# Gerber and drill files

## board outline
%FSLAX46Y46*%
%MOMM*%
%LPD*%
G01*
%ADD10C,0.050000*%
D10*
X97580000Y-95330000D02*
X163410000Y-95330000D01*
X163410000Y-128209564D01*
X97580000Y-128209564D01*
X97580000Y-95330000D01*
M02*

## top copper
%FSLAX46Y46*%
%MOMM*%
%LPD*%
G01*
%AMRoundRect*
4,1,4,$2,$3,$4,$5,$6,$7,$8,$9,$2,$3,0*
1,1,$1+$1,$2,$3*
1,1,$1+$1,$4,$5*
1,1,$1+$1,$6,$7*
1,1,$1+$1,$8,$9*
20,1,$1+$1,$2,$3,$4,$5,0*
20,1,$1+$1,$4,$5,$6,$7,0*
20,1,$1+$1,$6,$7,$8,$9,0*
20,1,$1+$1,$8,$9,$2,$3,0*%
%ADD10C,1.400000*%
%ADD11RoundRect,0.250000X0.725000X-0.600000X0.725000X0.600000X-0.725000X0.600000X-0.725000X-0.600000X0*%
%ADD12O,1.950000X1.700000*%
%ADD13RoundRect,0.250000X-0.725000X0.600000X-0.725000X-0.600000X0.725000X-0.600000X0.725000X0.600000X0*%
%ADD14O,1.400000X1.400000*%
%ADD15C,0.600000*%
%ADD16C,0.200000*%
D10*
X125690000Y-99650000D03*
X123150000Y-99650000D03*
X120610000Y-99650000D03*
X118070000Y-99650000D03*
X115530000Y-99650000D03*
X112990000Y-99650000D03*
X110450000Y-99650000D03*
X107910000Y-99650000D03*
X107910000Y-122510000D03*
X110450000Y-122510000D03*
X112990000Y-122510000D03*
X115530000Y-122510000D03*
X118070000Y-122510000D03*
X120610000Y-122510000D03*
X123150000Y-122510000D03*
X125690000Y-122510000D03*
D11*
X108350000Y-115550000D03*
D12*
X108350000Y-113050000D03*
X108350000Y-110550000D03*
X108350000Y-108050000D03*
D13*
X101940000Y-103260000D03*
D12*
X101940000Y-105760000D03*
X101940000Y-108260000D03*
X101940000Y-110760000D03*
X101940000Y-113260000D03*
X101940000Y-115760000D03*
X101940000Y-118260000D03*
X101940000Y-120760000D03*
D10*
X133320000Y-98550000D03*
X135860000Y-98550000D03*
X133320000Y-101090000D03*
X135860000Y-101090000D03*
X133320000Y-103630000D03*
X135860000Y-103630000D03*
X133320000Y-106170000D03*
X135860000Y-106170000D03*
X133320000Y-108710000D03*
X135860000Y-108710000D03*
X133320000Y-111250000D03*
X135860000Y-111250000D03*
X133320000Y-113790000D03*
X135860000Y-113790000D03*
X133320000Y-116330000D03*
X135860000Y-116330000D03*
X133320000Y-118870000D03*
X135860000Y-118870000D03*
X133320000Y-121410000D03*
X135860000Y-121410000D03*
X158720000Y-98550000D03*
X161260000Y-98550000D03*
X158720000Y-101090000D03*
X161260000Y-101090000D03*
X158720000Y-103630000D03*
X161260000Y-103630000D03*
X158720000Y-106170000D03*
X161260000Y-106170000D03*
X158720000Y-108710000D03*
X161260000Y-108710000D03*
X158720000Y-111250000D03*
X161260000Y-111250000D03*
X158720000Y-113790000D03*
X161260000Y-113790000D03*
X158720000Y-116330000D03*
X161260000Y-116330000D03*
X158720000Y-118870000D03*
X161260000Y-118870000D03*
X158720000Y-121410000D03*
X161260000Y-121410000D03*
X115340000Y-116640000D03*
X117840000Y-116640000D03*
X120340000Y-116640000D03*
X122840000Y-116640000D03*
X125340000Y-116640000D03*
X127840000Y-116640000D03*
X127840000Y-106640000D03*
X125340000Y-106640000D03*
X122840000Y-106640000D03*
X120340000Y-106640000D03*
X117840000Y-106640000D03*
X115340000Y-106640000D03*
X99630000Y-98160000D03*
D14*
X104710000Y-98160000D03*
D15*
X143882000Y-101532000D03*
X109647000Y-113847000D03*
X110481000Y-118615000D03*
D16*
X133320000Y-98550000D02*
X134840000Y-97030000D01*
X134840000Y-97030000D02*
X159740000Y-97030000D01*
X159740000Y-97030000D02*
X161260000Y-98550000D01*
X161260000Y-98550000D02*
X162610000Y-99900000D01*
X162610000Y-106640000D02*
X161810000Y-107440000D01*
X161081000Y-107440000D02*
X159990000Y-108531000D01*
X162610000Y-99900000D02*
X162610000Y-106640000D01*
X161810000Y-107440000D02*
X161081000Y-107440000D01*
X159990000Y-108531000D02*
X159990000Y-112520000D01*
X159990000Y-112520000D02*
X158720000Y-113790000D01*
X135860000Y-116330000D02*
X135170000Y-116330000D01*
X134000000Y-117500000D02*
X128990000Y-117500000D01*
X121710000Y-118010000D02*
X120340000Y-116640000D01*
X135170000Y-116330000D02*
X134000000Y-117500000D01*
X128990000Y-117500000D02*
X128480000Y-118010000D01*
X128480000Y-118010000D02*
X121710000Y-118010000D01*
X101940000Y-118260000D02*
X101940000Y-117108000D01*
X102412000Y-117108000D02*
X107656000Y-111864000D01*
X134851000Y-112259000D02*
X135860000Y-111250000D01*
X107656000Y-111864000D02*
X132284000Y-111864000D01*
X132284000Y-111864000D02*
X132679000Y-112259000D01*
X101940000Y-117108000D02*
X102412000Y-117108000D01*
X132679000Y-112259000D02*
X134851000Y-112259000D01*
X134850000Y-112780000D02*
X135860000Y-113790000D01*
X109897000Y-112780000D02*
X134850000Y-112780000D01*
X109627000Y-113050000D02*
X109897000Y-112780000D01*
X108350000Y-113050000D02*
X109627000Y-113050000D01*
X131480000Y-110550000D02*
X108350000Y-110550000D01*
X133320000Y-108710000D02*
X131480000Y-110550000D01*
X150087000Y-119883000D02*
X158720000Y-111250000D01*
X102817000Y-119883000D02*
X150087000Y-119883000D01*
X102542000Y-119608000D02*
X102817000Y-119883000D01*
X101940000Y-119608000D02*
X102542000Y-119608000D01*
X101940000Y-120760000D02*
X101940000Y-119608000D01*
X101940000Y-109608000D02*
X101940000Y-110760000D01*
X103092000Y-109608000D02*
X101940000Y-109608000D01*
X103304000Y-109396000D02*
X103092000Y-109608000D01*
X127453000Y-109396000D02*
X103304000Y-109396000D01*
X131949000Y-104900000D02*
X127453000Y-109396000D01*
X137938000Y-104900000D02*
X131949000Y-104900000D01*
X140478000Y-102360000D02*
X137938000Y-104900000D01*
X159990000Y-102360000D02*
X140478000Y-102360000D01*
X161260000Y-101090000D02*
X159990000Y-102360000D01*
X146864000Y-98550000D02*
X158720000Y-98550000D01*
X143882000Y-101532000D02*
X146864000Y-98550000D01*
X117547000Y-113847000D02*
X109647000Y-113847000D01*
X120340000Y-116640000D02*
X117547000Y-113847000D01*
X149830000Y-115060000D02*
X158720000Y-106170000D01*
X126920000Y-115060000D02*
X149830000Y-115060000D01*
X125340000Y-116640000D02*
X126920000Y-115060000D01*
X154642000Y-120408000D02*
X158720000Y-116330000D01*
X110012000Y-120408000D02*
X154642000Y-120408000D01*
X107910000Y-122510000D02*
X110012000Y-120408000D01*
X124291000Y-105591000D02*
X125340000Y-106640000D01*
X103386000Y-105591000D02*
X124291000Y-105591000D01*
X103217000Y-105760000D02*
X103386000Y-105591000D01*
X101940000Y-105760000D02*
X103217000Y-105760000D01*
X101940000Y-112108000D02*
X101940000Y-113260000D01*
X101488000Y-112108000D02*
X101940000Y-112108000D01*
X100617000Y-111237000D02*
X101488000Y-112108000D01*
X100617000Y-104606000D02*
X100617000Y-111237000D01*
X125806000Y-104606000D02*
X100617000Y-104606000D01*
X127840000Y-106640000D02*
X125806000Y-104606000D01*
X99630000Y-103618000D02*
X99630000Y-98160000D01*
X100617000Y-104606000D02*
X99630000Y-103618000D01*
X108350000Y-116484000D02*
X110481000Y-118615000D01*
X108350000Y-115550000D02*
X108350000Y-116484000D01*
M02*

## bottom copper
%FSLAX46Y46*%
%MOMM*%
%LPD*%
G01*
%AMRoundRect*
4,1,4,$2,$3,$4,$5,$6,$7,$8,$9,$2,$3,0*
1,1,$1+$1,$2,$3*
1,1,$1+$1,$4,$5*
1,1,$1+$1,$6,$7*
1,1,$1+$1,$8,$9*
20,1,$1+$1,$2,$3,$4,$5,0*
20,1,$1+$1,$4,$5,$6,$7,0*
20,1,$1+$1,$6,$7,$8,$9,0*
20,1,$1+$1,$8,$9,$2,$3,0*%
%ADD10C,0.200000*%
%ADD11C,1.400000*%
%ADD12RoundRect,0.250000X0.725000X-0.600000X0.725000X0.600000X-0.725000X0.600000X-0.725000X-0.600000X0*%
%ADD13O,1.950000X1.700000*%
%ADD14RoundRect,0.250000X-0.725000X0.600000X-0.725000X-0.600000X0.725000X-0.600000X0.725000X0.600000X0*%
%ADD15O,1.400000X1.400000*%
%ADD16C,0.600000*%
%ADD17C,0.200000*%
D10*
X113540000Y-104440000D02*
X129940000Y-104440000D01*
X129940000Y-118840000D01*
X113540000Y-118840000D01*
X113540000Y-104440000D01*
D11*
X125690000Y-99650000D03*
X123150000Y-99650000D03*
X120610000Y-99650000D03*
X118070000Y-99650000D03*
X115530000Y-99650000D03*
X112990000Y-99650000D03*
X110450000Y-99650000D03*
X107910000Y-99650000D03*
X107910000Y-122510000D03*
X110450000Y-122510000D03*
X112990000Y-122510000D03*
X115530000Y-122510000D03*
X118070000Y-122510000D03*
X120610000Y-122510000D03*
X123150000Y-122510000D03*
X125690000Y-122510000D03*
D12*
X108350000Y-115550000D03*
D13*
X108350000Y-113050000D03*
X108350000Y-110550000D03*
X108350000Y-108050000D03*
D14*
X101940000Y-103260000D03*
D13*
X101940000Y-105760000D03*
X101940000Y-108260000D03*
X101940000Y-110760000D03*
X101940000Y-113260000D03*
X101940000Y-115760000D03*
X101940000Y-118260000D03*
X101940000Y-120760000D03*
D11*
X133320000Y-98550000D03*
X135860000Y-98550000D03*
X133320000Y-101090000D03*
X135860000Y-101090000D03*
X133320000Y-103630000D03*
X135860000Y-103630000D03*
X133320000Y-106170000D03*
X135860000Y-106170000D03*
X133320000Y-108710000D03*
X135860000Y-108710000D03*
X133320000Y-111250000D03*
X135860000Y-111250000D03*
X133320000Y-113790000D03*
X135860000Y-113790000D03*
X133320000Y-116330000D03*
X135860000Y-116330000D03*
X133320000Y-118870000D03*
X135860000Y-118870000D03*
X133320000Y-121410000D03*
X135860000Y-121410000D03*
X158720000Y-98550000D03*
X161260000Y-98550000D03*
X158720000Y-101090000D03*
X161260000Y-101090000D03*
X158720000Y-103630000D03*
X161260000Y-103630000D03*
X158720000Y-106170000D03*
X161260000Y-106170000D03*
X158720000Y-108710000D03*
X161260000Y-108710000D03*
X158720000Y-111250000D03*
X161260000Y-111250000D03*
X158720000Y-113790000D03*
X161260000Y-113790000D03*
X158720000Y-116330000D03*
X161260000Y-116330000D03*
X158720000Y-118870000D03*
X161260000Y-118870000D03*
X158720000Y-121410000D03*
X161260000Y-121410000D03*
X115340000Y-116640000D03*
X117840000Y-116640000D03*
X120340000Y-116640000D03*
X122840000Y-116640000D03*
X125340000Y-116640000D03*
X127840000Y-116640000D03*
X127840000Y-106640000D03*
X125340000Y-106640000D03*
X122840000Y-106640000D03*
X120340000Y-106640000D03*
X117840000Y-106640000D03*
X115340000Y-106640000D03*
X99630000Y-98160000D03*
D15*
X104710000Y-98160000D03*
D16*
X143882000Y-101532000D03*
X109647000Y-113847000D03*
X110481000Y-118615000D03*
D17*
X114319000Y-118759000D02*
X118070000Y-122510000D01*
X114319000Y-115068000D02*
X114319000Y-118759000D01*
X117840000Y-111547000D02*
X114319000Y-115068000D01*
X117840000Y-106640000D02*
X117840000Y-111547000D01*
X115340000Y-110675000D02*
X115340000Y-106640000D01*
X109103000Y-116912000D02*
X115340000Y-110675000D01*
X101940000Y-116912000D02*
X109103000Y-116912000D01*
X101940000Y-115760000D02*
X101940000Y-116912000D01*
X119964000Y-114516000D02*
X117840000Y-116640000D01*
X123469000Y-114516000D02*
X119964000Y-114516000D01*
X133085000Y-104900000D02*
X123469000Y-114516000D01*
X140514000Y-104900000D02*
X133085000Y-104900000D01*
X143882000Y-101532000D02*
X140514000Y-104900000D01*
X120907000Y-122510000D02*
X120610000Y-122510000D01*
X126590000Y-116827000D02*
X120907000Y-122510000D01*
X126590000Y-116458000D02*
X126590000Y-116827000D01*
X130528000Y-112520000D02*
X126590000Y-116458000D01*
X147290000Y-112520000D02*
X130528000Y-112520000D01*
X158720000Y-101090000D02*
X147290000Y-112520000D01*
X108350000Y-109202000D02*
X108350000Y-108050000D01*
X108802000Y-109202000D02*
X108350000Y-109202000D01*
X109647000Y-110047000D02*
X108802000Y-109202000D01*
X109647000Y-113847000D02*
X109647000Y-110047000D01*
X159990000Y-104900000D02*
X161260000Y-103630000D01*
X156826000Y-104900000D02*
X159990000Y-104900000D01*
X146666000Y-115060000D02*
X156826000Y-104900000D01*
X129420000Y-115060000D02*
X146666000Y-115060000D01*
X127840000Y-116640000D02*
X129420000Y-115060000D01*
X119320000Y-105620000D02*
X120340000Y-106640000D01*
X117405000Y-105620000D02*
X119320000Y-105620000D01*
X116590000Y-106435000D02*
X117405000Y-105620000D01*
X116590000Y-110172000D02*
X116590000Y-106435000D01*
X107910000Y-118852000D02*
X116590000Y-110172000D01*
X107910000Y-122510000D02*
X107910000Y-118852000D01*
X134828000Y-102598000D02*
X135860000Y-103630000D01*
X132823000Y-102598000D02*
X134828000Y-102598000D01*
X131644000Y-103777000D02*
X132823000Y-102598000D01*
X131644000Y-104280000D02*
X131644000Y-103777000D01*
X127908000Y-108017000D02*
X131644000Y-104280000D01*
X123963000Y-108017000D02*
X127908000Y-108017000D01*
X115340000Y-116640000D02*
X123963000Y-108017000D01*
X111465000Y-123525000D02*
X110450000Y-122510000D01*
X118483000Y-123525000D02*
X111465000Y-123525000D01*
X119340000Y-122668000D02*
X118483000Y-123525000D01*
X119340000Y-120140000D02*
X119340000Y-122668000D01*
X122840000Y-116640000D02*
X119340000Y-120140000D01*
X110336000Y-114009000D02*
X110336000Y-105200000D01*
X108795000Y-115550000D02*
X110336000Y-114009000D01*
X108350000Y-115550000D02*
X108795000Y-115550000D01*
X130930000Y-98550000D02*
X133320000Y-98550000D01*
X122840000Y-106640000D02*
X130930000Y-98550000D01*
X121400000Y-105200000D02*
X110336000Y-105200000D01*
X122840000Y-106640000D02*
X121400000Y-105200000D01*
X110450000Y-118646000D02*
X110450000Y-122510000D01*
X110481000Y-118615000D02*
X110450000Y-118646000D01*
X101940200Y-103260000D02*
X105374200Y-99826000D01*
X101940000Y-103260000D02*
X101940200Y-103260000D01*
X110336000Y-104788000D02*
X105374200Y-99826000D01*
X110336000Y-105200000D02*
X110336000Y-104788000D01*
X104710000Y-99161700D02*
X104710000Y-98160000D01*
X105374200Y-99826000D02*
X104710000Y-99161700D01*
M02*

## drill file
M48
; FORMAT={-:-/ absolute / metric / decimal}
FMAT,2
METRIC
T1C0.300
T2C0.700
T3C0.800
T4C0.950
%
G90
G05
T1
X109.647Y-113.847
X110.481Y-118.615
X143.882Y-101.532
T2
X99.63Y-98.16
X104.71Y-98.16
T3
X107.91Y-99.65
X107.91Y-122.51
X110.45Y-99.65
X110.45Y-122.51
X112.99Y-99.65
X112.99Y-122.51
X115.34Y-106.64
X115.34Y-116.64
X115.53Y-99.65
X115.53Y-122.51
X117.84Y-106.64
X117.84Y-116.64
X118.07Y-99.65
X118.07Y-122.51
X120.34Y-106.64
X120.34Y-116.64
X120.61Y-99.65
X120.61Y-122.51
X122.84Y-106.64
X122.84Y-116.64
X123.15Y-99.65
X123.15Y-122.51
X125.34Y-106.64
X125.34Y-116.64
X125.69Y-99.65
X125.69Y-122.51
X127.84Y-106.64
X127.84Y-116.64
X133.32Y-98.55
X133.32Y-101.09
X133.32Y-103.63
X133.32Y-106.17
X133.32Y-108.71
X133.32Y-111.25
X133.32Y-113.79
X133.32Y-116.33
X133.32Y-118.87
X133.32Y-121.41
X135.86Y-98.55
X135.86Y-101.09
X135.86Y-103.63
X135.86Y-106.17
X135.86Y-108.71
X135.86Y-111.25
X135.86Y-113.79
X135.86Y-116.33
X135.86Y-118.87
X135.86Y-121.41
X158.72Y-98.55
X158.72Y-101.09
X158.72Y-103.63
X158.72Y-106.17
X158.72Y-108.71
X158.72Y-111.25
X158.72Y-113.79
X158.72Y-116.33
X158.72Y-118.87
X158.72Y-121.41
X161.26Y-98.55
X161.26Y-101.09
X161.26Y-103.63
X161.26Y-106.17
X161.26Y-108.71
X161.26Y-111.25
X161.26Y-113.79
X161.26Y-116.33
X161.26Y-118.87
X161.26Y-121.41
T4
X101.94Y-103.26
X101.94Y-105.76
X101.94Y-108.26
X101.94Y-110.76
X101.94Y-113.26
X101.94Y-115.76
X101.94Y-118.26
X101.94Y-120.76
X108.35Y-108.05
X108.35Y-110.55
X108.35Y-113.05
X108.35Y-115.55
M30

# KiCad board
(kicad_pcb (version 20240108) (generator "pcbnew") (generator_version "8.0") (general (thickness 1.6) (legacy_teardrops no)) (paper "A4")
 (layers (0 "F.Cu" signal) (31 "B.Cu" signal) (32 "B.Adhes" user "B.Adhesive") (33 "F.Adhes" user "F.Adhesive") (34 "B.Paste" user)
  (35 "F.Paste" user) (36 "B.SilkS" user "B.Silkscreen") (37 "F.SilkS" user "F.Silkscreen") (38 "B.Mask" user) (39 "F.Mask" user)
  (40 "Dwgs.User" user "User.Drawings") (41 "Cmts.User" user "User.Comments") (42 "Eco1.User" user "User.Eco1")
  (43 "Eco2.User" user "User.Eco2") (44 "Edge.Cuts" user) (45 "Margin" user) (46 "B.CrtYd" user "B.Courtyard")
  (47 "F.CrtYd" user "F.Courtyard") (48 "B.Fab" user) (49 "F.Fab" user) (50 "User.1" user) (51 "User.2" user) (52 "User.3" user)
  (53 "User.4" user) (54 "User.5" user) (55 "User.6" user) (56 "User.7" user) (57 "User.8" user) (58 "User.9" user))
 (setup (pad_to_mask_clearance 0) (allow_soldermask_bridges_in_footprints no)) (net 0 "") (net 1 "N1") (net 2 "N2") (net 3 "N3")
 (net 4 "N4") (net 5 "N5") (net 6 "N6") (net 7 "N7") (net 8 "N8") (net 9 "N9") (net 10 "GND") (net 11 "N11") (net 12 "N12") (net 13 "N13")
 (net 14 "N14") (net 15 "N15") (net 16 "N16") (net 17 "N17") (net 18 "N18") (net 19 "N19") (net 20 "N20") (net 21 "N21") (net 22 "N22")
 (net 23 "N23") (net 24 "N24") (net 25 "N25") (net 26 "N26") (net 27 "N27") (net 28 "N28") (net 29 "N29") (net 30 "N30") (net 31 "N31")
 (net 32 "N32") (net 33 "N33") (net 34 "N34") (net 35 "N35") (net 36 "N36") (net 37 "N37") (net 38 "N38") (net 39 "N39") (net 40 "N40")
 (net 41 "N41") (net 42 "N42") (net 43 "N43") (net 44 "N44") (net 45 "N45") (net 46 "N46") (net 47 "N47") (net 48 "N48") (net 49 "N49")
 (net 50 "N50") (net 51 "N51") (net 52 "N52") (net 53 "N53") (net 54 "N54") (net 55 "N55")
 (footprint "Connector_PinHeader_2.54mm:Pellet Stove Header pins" (layer "F.Cu") (at 114.26 111.08 -90)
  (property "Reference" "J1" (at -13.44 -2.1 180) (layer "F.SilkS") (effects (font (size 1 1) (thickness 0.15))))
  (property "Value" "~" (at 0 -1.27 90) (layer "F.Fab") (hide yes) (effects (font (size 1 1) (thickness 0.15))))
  (pad "1" thru_hole circle (at -11.43 -11.43 180) (size 1.4 1.4) (drill 0.8) (layers "*.Cu" "*.Mask") (remove_unused_layers no)
   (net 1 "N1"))
  (pad "2" thru_hole circle (at -11.43 -8.89 180) (size 1.4 1.4) (drill 0.8) (layers "*.Cu" "*.Mask") (remove_unused_layers no) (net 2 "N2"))
  (pad "3" thru_hole circle (at -11.43 -6.35 180) (size 1.4 1.4) (drill 0.8) (layers "*.Cu" "*.Mask") (remove_unused_layers no) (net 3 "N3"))
  (pad "4" thru_hole circle (at -11.43 -3.81 180) (size 1.4 1.4) (drill 0.8) (layers "*.Cu" "*.Mask") (remove_unused_layers no) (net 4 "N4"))
  (pad "5" thru_hole circle (at -11.43 -1.27 180) (size 1.4 1.4) (drill 0.8) (layers "*.Cu" "*.Mask") (remove_unused_layers no) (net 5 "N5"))
  (pad "6" thru_hole circle (at -11.43 1.27 180) (size 1.4 1.4) (drill 0.8) (layers "*.Cu" "*.Mask") (remove_unused_layers no) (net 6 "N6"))
  (pad "7" thru_hole circle (at -11.43 3.81 180) (size 1.4 1.4) (drill 0.8) (layers "*.Cu" "*.Mask") (remove_unused_layers no) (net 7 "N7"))
  (pad "8" thru_hole circle (at -11.43 6.35 180) (size 1.4 1.4) (drill 0.8) (layers "*.Cu" "*.Mask") (remove_unused_layers no) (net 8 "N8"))
  (pad "9" thru_hole circle (at 11.43 6.35 180) (size 1.4 1.4) (drill 0.8) (layers "*.Cu" "*.Mask") (remove_unused_layers no) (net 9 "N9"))
  (pad "10" thru_hole circle (at 11.43 3.81 180) (size 1.4 1.4) (drill 0.8) (layers "*.Cu" "*.Mask") (remove_unused_layers no)
   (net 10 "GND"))
  (pad "11" thru_hole circle (at 11.43 1.27 180) (size 1.4 1.4) (drill 0.8) (layers "*.Cu" "*.Mask") (remove_unused_layers no)
   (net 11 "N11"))
  (pad "12" thru_hole circle (at 11.43 -1.27 180) (size 1.4 1.4) (drill 0.8) (layers "*.Cu" "*.Mask") (remove_unused_layers no)
   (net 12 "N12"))
  (pad "13" thru_hole circle (at 11.43 -3.81 180) (size 1.4 1.4) (drill 0.8) (layers "*.Cu" "*.Mask") (remove_unused_layers no)
   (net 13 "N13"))
  (pad "14" thru_hole circle (at 11.43 -6.35 180) (size 1.4 1.4) (drill 0.8) (layers "*.Cu" "*.Mask") (remove_unused_layers no)
   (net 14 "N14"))
  (pad "15" thru_hole circle (at 11.43 -8.89 180) (size 1.4 1.4) (drill 0.8) (layers "*.Cu" "*.Mask") (remove_unused_layers no)
   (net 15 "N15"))
  (pad "16" thru_hole circle (at 11.43 -11.43 180) (size 1.4 1.4) (drill 0.8) (layers "*.Cu" "*.Mask") (remove_unused_layers no)
   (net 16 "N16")))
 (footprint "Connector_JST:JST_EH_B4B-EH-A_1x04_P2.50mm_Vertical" (layer "F.Cu") (at 108.35 115.55 90)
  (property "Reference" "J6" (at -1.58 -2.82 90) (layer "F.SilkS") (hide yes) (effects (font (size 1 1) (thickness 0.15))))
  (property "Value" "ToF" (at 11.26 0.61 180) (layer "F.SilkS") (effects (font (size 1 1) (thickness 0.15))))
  (pad "1" thru_hole roundrect (at 0 0 90) (size 1.7 1.95) (drill 0.95) (layers "*.Cu" "*.Mask") (remove_unused_layers no)
   (roundrect_rratio 0.147059) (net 10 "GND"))
  (pad "2" thru_hole oval (at 2.5 0 90) (size 1.7 1.95) (drill 0.95) (layers "*.Cu" "*.Mask") (remove_unused_layers no) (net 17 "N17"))
  (pad "3" thru_hole oval (at 5 0 90) (size 1.7 1.95) (drill 0.95) (layers "*.Cu" "*.Mask") (remove_unused_layers no) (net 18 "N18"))
  (pad "4" thru_hole oval (at 7.5 0 90) (size 1.7 1.95) (drill 0.95) (layers "*.Cu" "*.Mask") (remove_unused_layers no) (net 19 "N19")))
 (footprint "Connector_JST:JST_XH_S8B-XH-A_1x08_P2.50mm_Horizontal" (layer "F.Cu") (at 101.94 103.26 -90)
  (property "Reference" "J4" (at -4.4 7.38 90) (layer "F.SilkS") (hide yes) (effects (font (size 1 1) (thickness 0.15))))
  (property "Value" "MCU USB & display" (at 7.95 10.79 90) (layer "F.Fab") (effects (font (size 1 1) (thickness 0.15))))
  (pad "1" thru_hole roundrect (at 0 0 270) (size 1.7 1.95) (drill 0.95) (layers "*.Cu" "*.Mask") (remove_unused_layers no)
   (roundrect_rratio 0.147059) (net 10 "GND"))
  (pad "2" thru_hole oval (at 2.5 0 270) (size 1.7 1.95) (drill 0.95) (layers "*.Cu" "*.Mask") (remove_unused_layers no) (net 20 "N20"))
  (pad "3" thru_hole oval (at 5 0 270) (size 1.7 1.95) (drill 0.95) (layers "*.Cu" "*.Mask") (remove_unused_layers no) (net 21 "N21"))
  (pad "4" thru_hole oval (at 7.5 0 270) (size 1.7 1.95) (drill 0.95) (layers "*.Cu" "*.Mask") (remove_unused_layers no) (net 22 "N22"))
  (pad "5" thru_hole oval (at 10 0 270) (size 1.7 1.95) (drill 0.95) (layers "*.Cu" "*.Mask") (remove_unused_layers no) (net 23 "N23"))
  (pad "6" thru_hole oval (at 12.5 0 270) (size 1.7 1.95) (drill 0.95) (layers "*.Cu" "*.Mask") (remove_unused_layers no) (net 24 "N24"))
  (pad "7" thru_hole oval (at 15 0 270) (size 1.7 1.95) (drill 0.95) (layers "*.Cu" "*.Mask") (remove_unused_layers no) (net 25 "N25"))
  (pad "8" thru_hole oval (at 17.5 0 270) (size 1.7 1.95) (drill 0.95) (layers "*.Cu" "*.Mask") (remove_unused_layers no) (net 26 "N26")))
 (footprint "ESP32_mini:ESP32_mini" (layer "F.Cu") (at 147.29 109.98)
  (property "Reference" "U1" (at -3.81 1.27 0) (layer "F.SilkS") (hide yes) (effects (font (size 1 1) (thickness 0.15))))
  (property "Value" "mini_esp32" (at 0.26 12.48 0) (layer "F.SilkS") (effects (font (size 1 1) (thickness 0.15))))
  (pad "1" thru_hole circle (at -13.97 -11.43 270) (size 1.4 1.4) (drill 0.8) (layers "*.Cu" "*.Mask") (remove_unused_layers no)
   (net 10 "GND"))
  (pad "2" thru_hole circle (at -11.43 -11.43 270) (size 1.4 1.4) (drill 0.8) (layers "*.Cu" "*.Mask") (remove_unused_layers no)
   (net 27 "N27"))
  (pad "3" thru_hole circle (at -13.97 -8.89 270) (size 1.4 1.4) (drill 0.8) (layers "*.Cu" "*.Mask") (remove_unused_layers no)
   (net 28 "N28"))
  (pad "4" thru_hole circle (at -11.43 -8.89 270) (size 1.4 1.4) (drill 0.8) (layers "*.Cu" "*.Mask") (remove_unused_layers no)
   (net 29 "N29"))
  (pad "5" thru_hole circle (at -13.97 -6.35 270) (size 1.4 1.4) (drill 0.8) (layers "*.Cu" "*.Mask") (remove_unused_layers no)
   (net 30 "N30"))
  (pad "6" thru_hole circle (at -11.43 -6.35 270) (size 1.4 1.4) (drill 0.8) (layers "*.Cu" "*.Mask") (remove_unused_layers no)
   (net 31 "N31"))
  (pad "7" thru_hole circle (at -13.97 -3.81 270) (size 1.4 1.4) (drill 0.8) (layers "*.Cu" "*.Mask") (remove_unused_layers no)
   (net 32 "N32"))
  (pad "8" thru_hole circle (at -11.43 -3.81 270) (size 1.4 1.4) (drill 0.8) (layers "*.Cu" "*.Mask") (remove_unused_layers no)
   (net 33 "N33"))
  (pad "9" thru_hole circle (at -13.97 -1.27 270) (size 1.4 1.4) (drill 0.8) (layers "*.Cu" "*.Mask") (remove_unused_layers no)
   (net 18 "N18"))
  (pad "10" thru_hole circle (at -11.43 -1.27 270) (size 1.4 1.4) (drill 0.8) (layers "*.Cu" "*.Mask") (remove_unused_layers no)
   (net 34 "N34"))
  (pad "11" thru_hole circle (at -13.97 1.27 270) (size 1.4 1.4) (drill 0.8) (layers "*.Cu" "*.Mask") (remove_unused_layers no)
   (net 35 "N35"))
  (pad "12" thru_hole circle (at -11.43 1.27 270) (size 1.4 1.4) (drill 0.8) (layers "*.Cu" "*.Mask") (remove_unused_layers no)
   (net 25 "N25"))
  (pad "13" thru_hole circle (at -13.97 3.81 270) (size 1.4 1.4) (drill 0.8) (layers "*.Cu" "*.Mask") (remove_unused_layers no)
   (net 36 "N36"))
  (pad "14" thru_hole circle (at -11.43 3.81 270) (size 1.4 1.4) (drill 0.8) (layers "*.Cu" "*.Mask") (remove_unused_layers no)
   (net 17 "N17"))
  (pad "15" thru_hole circle (at -13.97 6.35 270) (size 1.4 1.4) (drill 0.8) (layers "*.Cu" "*.Mask") (remove_unused_layers no)
   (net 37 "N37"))
  (pad "16" thru_hole circle (at -11.43 6.35 270) (size 1.4 1.4) (drill 0.8) (layers "*.Cu" "*.Mask") (remove_unused_layers no)
   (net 19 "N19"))
  (pad "17" thru_hole circle (at -13.97 8.89 270) (size 1.4 1.4) (drill 0.8) (layers "*.Cu" "*.Mask") (remove_unused_layers no)
   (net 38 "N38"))
  (pad "18" thru_hole circle (at -11.43 8.89 270) (size 1.4 1.4) (drill 0.8) (layers "*.Cu" "*.Mask") (remove_unused_layers no)
   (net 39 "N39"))
  (pad "19" thru_hole circle (at -13.97 11.43 270) (size 1.4 1.4) (drill 0.8) (layers "*.Cu" "*.Mask") (remove_unused_layers no)
   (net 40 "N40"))
  (pad "20" thru_hole circle (at -11.43 11.43 270) (size 1.4 1.4) (drill 0.8) (layers "*.Cu" "*.Mask") (remove_unused_layers no)
   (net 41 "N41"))
  (pad "21" thru_hole circle (at 11.43 -11.43 270) (size 1.4 1.4) (drill 0.8) (layers "*.Cu" "*.Mask") (remove_unused_layers no)
   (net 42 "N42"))
  (pad "22" thru_hole circle (at 13.97 -11.43 270) (size 1.4 1.4) (drill 0.8) (layers "*.Cu" "*.Mask") (remove_unused_layers no)
   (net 10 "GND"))
  (pad "23" thru_hole circle (at 11.43 -8.89 270) (size 1.4 1.4) (drill 0.8) (layers "*.Cu" "*.Mask") (remove_unused_layers no)
   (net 14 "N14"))
  (pad "24" thru_hole circle (at 13.97 -8.89 270) (size 1.4 1.4) (drill 0.8) (layers "*.Cu" "*.Mask") (remove_unused_layers no)
   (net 22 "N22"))
  (pad "25" thru_hole circle (at 11.43 -6.35 270) (size 1.4 1.4) (drill 0.8) (layers "*.Cu" "*.Mask") (remove_unused_layers no)
   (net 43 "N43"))
  (pad "26" thru_hole circle (at 13.97 -6.35 270) (size 1.4 1.4) (drill 0.8) (layers "*.Cu" "*.Mask") (remove_unused_layers no)
   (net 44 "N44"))
  (pad "27" thru_hole circle (at 11.43 -3.81 270) (size 1.4 1.4) (drill 0.8) (layers "*.Cu" "*.Mask") (remove_unused_layers no)
   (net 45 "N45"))
  (pad "28" thru_hole circle (at 13.97 -3.81 270) (size 1.4 1.4) (drill 0.8) (layers "*.Cu" "*.Mask") (remove_unused_layers no)
   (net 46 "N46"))
  (pad "29" thru_hole circle (at 11.43 -1.27 270) (size 1.4 1.4) (drill 0.8) (layers "*.Cu" "*.Mask") (remove_unused_layers no)
   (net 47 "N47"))
  (pad "30" thru_hole circle (at 13.97 -1.27 270) (size 1.4 1.4) (drill 0.8) (layers "*.Cu" "*.Mask") (remove_unused_layers no)
   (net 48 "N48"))
  (pad "31" thru_hole circle (at 11.43 1.27 270) (size 1.4 1.4) (drill 0.8) (layers "*.Cu" "*.Mask") (remove_unused_layers no)
   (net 26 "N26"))
  (pad "32" thru_hole circle (at 13.97 1.27 270) (size 1.4 1.4) (drill 0.8) (layers "*.Cu" "*.Mask") (remove_unused_layers no)
   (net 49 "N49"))
  (pad "33" thru_hole circle (at 11.43 3.81 270) (size 1.4 1.4) (drill 0.8) (layers "*.Cu" "*.Mask") (remove_unused_layers no)
   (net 10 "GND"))
  (pad "34" thru_hole circle (at 13.97 3.81 270) (size 1.4 1.4) (drill 0.8) (layers "*.Cu" "*.Mask") (remove_unused_layers no)
   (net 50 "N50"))
  (pad "35" thru_hole circle (at 11.43 6.35 270) (size 1.4 1.4) (drill 0.8) (layers "*.Cu" "*.Mask") (remove_unused_layers no) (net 9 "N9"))
  (pad "36" thru_hole circle (at 13.97 6.35 270) (size 1.4 1.4) (drill 0.8) (layers "*.Cu" "*.Mask") (remove_unused_layers no)
   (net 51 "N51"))
  (pad "37" thru_hole circle (at 11.43 8.89 270) (size 1.4 1.4) (drill 0.8) (layers "*.Cu" "*.Mask") (remove_unused_layers no)
   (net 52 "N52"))
  (pad "38" thru_hole circle (at 13.97 8.89 270) (size 1.4 1.4) (drill 0.8) (layers "*.Cu" "*.Mask") (remove_unused_layers no)
   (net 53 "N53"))
  (pad "39" thru_hole circle (at 11.43 11.43 270) (size 1.4 1.4) (drill 0.8) (layers "*.Cu" "*.Mask") (remove_unused_layers no)
   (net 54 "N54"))
  (pad "40" thru_hole circle (at 13.97 11.43 270) (size 1.4 1.4) (drill 0.8) (layers "*.Cu" "*.Mask") (remove_unused_layers no)
   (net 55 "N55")))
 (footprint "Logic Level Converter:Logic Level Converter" (layer "F.Cu") (at 123.54 113.04)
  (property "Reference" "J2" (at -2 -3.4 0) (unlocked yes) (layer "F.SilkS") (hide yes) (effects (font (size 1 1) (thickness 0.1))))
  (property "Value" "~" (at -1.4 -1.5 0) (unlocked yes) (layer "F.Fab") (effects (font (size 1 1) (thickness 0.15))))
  (fp_rect (start -10 -8.6) (end 6.4 5.8) (stroke (width 0.2) (type default)) (fill none) (layer "B.Cu"))
  (pad "1" thru_hole circle (at -8.2 3.6 270) (size 1.4 1.4) (drill 0.8) (layers "*.Cu" "*.Mask") (remove_unused_layers no) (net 31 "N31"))
  (pad "2" thru_hole circle (at -5.7 3.6 270) (size 1.4 1.4) (drill 0.8) (layers "*.Cu" "*.Mask") (remove_unused_layers no) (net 42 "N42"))
  (pad "3" thru_hole circle (at -3.2 3.6 270) (size 1.4 1.4) (drill 0.8) (layers "*.Cu" "*.Mask") (remove_unused_layers no) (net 19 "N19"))
  (pad "4" thru_hole circle (at -0.7 3.6 270) (size 1.4 1.4) (drill 0.8) (layers "*.Cu" "*.Mask") (remove_unused_layers no) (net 10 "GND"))
  (pad "5" thru_hole circle (at 1.8 3.6 270) (size 1.4 1.4) (drill 0.8) (layers "*.Cu" "*.Mask") (remove_unused_layers no) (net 45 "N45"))
  (pad "6" thru_hole circle (at 4.3 3.6 270) (size 1.4 1.4) (drill 0.8) (layers "*.Cu" "*.Mask") (remove_unused_layers no) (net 44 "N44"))
  (pad "7" thru_hole circle (at 4.3 -6.4 270) (size 1.4 1.4) (drill 0.8) (layers "*.Cu" "*.Mask") (remove_unused_layers no) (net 23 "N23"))
  (pad "8" thru_hole circle (at 1.8 -6.4 270) (size 1.4 1.4) (drill 0.8) (layers "*.Cu" "*.Mask") (remove_unused_layers no) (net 20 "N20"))
  (pad "9" thru_hole circle (at -0.7 -6.4 270) (size 1.4 1.4) (drill 0.8) (layers "*.Cu" "*.Mask") (remove_unused_layers no) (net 10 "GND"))
  (pad "10" thru_hole circle (at -3.2 -6.4 270) (size 1.4 1.4) (drill 0.8) (layers "*.Cu" "*.Mask") (remove_unused_layers no) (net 9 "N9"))
  (pad "11" thru_hole circle (at -5.7 -6.4 270) (size 1.4 1.4) (drill 0.8) (layers "*.Cu" "*.Mask") (remove_unused_layers no) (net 13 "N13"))
  (pad "12" thru_hole circle (at -8.2 -6.4 270) (size 1.4 1.4) (drill 0.8) (layers "*.Cu" "*.Mask") (remove_unused_layers no) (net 24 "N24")))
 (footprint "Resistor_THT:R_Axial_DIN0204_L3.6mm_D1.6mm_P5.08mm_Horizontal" (layer "F.Cu") (at 99.63 98.16)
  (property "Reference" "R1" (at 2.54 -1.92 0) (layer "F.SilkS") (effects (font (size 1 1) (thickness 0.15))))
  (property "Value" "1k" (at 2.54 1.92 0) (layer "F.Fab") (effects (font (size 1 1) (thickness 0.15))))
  (pad "1" thru_hole circle (at 0 0) (size 1.4 1.4) (drill 0.7) (layers "*.Cu" "*.Mask") (remove_unused_layers no) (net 23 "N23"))
  (pad "2" thru_hole oval (at 5.08 0) (size 1.4 1.4) (drill 0.7) (layers "*.Cu" "*.Mask") (remove_unused_layers no) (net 10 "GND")))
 (gr_rect (start 97.58 95.33) (end 163.41 128.209564) (stroke (width 0.05) (type default)) (fill none) (layer "Edge.Cuts"))
 (segment (start 133.32 98.55) (end 134.84 97.03) (width 0.2) (layer "F.Cu") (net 10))
 (segment (start 134.84 97.03) (end 159.74 97.03) (width 0.2) (layer "F.Cu") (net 10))
 (segment (start 159.74 97.03) (end 161.26 98.55) (width 0.2) (layer "F.Cu") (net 10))
 (segment (start 161.081 107.44) (end 159.99 108.531) (width 0.2) (layer "F.Cu") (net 10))
 (segment (start 159.99 108.531) (end 159.99 112.52) (width 0.2) (layer "F.Cu") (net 10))
 (segment (start 162.61 106.64) (end 161.81 107.44) (width 0.2) (layer "F.Cu") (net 10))
 (segment (start 159.99 112.52) (end 158.72 113.79) (width 0.2) (layer "F.Cu") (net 10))
 (segment (start 161.26 98.55) (end 162.61 99.9) (width 0.2) (layer "F.Cu") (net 10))
 (segment (start 108.35 116.484) (end 110.481 118.615) (width 0.2) (layer "F.Cu") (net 10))
 (segment (start 162.61 99.9) (end 162.61 106.64) (width 0.2) (layer "F.Cu") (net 10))
 (segment (start 161.81 107.44) (end 161.081 107.44) (width 0.2) (layer "F.Cu") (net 10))
 (segment (start 108.35 115.55) (end 108.35 116.484) (width 0.2) (layer "F.Cu") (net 10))
 (via (at 110.481 118.615) (size 0.6) (drill 0.3) (layers "F.Cu" "B.Cu") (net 10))
 (segment (start 119.34 120.14) (end 119.34 122.668) (width 0.2) (layer "B.Cu") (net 10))
 (segment (start 122.84 106.64) (end 130.93 98.55) (width 0.2) (layer "B.Cu") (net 10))
 (segment (start 105.3742 99.826) (end 104.71 99.1617) (width 0.2) (layer "B.Cu") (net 10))
 (segment (start 119.34 122.668) (end 118.483 123.525) (width 0.2) (layer "B.Cu") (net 10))
 (segment (start 111.465 123.525) (end 110.45 122.51) (width 0.2) (layer "B.Cu") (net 10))
 (segment (start 108.795 115.55) (end 110.336 114.009) (width 0.2) (layer "B.Cu") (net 10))
 (segment (start 121.4 105.2) (end 110.336 105.2) (width 0.2) (layer "B.Cu") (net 10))
 (segment (start 101.9402 103.26) (end 105.3742 99.826) (width 0.2) (layer "B.Cu") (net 10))
 (segment (start 108.35 115.55) (end 108.795 115.55) (width 0.2) (layer "B.Cu") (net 10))
 (segment (start 110.336 105.2) (end 110.336 104.788) (width 0.2) (layer "B.Cu") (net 10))
 (segment (start 101.94 103.26) (end 101.9402 103.26) (width 0.2) (layer "B.Cu") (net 10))
 (segment (start 110.336 104.788) (end 105.3742 99.826) (width 0.2) (layer "B.Cu") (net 10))
 (segment (start 118.483 123.525) (end 111.465 123.525) (width 0.2) (layer "B.Cu") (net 10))
 (segment (start 104.71 99.1617) (end 104.71 98.16) (width 0.2) (layer "B.Cu") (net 10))
 (segment (start 122.84 116.64) (end 119.34 120.14) (width 0.2) (layer "B.Cu") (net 10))
 (segment (start 110.481 118.615) (end 110.45 118.646) (width 0.2) (layer "B.Cu") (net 10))
 (segment (start 110.336 114.009) (end 110.336 105.2) (width 0.2) (layer "B.Cu") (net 10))
 (segment (start 130.93 98.55) (end 133.32 98.55) (width 0.2) (layer "B.Cu") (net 10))
 (segment (start 110.45 118.646) (end 110.45 122.51) (width 0.2) (layer "B.Cu") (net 10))
 (segment (start 122.84 106.64) (end 121.4 105.2) (width 0.2) (layer "B.Cu") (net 10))
 (segment (start 100.617 104.606) (end 99.63 103.618) (width 0.2) (layer "F.Cu") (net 23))
 (segment (start 101.488 112.108) (end 101.94 112.108) (width 0.2) (layer "F.Cu") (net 23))
 (segment (start 125.806 104.606) (end 100.617 104.606) (width 0.2) (layer "F.Cu") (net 23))
 (segment (start 100.617 111.237) (end 101.488 112.108) (width 0.2) (layer "F.Cu") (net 23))
 (segment (start 99.63 103.618) (end 99.63 98.16) (width 0.2) (layer "F.Cu") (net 23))
 (segment (start 127.84 106.64) (end 125.806 104.606) (width 0.2) (layer "F.Cu") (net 23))
 (segment (start 100.617 104.606) (end 100.617 111.237) (width 0.2) (layer "F.Cu") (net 23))
 (segment (start 101.94 112.108) (end 101.94 113.26) (width 0.2) (layer "F.Cu") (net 23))
 (segment (start 101.94 105.76) (end 103.217 105.76) (width 0.2) (layer "F.Cu") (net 20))
 (segment (start 103.386 105.591) (end 124.291 105.591) (width 0.2) (layer "F.Cu") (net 20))
 (segment (start 124.291 105.591) (end 125.34 106.64) (width 0.2) (layer "F.Cu") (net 20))
 (segment (start 103.217 105.76) (end 103.386 105.591) (width 0.2) (layer "F.Cu") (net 20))
 (segment (start 123.963 108.017) (end 127.908 108.017) (width 0.2) (layer "B.Cu") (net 31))
 (segment (start 131.644 103.777) (end 132.823 102.598) (width 0.2) (layer "B.Cu") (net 31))
 (segment (start 115.34 116.64) (end 123.963 108.017) (width 0.2) (layer "B.Cu") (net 31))
 (segment (start 134.828 102.598) (end 135.86 103.63) (width 0.2) (layer "B.Cu") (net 31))
 (segment (start 132.823 102.598) (end 134.828 102.598) (width 0.2) (layer "B.Cu") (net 31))
 (segment (start 131.644 104.28) (end 131.644 103.777) (width 0.2) (layer "B.Cu") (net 31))
 (segment (start 127.908 108.017) (end 131.644 104.28) (width 0.2) (layer "B.Cu") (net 31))
 (segment (start 110.012 120.408) (end 154.642 120.408) (width 0.2) (layer "F.Cu") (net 9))
 (segment (start 107.91 122.51) (end 110.012 120.408) (width 0.2) (layer "F.Cu") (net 9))
 (segment (start 154.642 120.408) (end 158.72 116.33) (width 0.2) (layer "F.Cu") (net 9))
 (segment (start 117.405 105.62) (end 119.32 105.62) (width 0.2) (layer "B.Cu") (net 9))
 (segment (start 107.91 122.51) (end 107.91 118.852) (width 0.2) (layer "B.Cu") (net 9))
 (segment (start 116.59 110.172) (end 116.59 106.435) (width 0.2) (layer "B.Cu") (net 9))
 (segment (start 107.91 118.852) (end 116.59 110.172) (width 0.2) (layer "B.Cu") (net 9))
 (segment (start 116.59 106.435) (end 117.405 105.62) (width 0.2) (layer "B.Cu") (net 9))
 (segment (start 119.32 105.62) (end 120.34 106.64) (width 0.2) (layer "B.Cu") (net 9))
 (segment (start 149.83 115.06) (end 158.72 106.17) (width 0.2) (layer "F.Cu") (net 45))
 (segment (start 125.34 116.64) (end 126.92 115.06) (width 0.2) (layer "F.Cu") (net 45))
 (segment (start 126.92 115.06) (end 149.83 115.06) (width 0.2) (layer "F.Cu") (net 45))
 (segment (start 129.42 115.06) (end 146.666 115.06) (width 0.2) (layer "B.Cu") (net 44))
 (segment (start 159.99 104.9) (end 161.26 103.63) (width 0.2) (layer "B.Cu") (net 44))
 (segment (start 156.826 104.9) (end 159.99 104.9) (width 0.2) (layer "B.Cu") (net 44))
 (segment (start 146.666 115.06) (end 156.826 104.9) (width 0.2) (layer "B.Cu") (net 44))
 (segment (start 127.84 116.64) (end 129.42 115.06) (width 0.2) (layer "B.Cu") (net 44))
 (segment (start 120.34 116.64) (end 117.547 113.847) (width 0.2) (layer "F.Cu") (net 19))
 (segment (start 128.99 117.5) (end 128.48 118.01) (width 0.2) (layer "F.Cu") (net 19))
 (segment (start 135.17 116.33) (end 134 117.5) (width 0.2) (layer "F.Cu") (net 19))
 (segment (start 135.86 116.33) (end 135.17 116.33) (width 0.2) (layer "F.Cu") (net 19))
 (segment (start 134 117.5) (end 128.99 117.5) (width 0.2) (layer "F.Cu") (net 19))
 (segment (start 128.48 118.01) (end 121.71 118.01) (width 0.2) (layer "F.Cu") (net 19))
 (segment (start 121.71 118.01) (end 120.34 116.64) (width 0.2) (layer "F.Cu") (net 19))
 (segment (start 117.547 113.847) (end 109.647 113.847) (width 0.2) (layer "F.Cu") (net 19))
 (via (at 109.647 113.847) (size 0.6) (drill 0.3) (layers "F.Cu" "B.Cu") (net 19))
 (segment (start 108.802 109.202) (end 108.35 109.202) (width 0.2) (layer "B.Cu") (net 19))
 (segment (start 109.647 113.847) (end 109.647 110.047) (width 0.2) (layer "B.Cu") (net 19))
 (segment (start 109.647 110.047) (end 108.802 109.202) (width 0.2) (layer "B.Cu") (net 19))
 (segment (start 108.35 109.202) (end 108.35 108.05) (width 0.2) (layer "B.Cu") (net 19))
 (segment (start 120.907 122.51) (end 120.61 122.51) (width 0.2) (layer "B.Cu") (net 14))
 (segment (start 147.29 112.52) (end 130.528 112.52) (width 0.2) (layer "B.Cu") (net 14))
 (segment (start 130.528 112.52) (end 126.59 116.458) (width 0.2) (layer "B.Cu") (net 14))
 (segment (start 158.72 101.09) (end 147.29 112.52) (width 0.2) (layer "B.Cu") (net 14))
 (segment (start 126.59 116.827) (end 120.907 122.51) (width 0.2) (layer "B.Cu") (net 14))
 (segment (start 126.59 116.458) (end 126.59 116.827) (width 0.2) (layer "B.Cu") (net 14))
 (segment (start 146.864 98.55) (end 158.72 98.55) (width 0.2) (layer "F.Cu") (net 42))
 (segment (start 143.882 101.532) (end 146.864 98.55) (width 0.2) (layer "F.Cu") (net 42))
 (via (at 143.882 101.532) (size 0.6) (drill 0.3) (layers "F.Cu" "B.Cu") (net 42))
 (segment (start 140.514 104.9) (end 133.085 104.9) (width 0.2) (layer "B.Cu") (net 42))
 (segment (start 143.882 101.532) (end 140.514 104.9) (width 0.2) (layer "B.Cu") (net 42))
 (segment (start 119.964 114.516) (end 117.84 116.64) (width 0.2) (layer "B.Cu") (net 42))
 (segment (start 123.469 114.516) (end 119.964 114.516) (width 0.2) (layer "B.Cu") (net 42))
 (segment (start 133.085 104.9) (end 123.469 114.516) (width 0.2) (layer "B.Cu") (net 42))
 (segment (start 101.94 115.76) (end 101.94 116.912) (width 0.2) (layer "B.Cu") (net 24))
 (segment (start 101.94 116.912) (end 109.103 116.912) (width 0.2) (layer "B.Cu") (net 24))
 (segment (start 109.103 116.912) (end 115.34 110.675) (width 0.2) (layer "B.Cu") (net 24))
 (segment (start 115.34 110.675) (end 115.34 106.64) (width 0.2) (layer "B.Cu") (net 24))
 (segment (start 140.478 102.36) (end 137.938 104.9) (width 0.2) (layer "F.Cu") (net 22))
 (segment (start 127.453 109.396) (end 103.304 109.396) (width 0.2) (layer "F.Cu") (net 22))
 (segment (start 159.99 102.36) (end 140.478 102.36) (width 0.2) (layer "F.Cu") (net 22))
 (segment (start 103.304 109.396) (end 103.092 109.608) (width 0.2) (layer "F.Cu") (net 22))
 (segment (start 137.938 104.9) (end 131.949 104.9) (width 0.2) (layer "F.Cu") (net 22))
 (segment (start 161.26 101.09) (end 159.99 102.36) (width 0.2) (layer "F.Cu") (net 22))
 (segment (start 103.092 109.608) (end 101.94 109.608) (width 0.2) (layer "F.Cu") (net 22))
 (segment (start 101.94 109.608) (end 101.94 110.76) (width 0.2) (layer "F.Cu") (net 22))
 (segment (start 131.949 104.9) (end 127.453 109.396) (width 0.2) (layer "F.Cu") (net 22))
 (segment (start 134.851 112.259) (end 135.86 111.25) (width 0.2) (layer "F.Cu") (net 25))
 (segment (start 102.412 117.108) (end 107.656 111.864) (width 0.2) (layer "F.Cu") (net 25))
 (segment (start 101.94 118.26) (end 101.94 117.108) (width 0.2) (layer "F.Cu") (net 25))
 (segment (start 107.656 111.864) (end 132.284 111.864) (width 0.2) (layer "F.Cu") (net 25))
 (segment (start 132.679 112.259) (end 134.851 112.259) (width 0.2) (layer "F.Cu") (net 25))
 (segment (start 132.284 111.864) (end 132.679 112.259) (width 0.2) (layer "F.Cu") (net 25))
 (segment (start 101.94 117.108) (end 102.412 117.108) (width 0.2) (layer "F.Cu") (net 25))
 (segment (start 101.94 120.76) (end 101.94 119.608) (width 0.2) (layer "F.Cu") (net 26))
 (segment (start 101.94 119.608) (end 102.542 119.608) (width 0.2) (layer "F.Cu") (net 26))
 (segment (start 150.087 119.883) (end 158.72 111.25) (width 0.2) (layer "F.Cu") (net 26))
 (segment (start 102.817 119.883) (end 150.087 119.883) (width 0.2) (layer "F.Cu") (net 26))
 (segment (start 102.542 119.608) (end 102.817 119.883) (width 0.2) (layer "F.Cu") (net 26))
 (segment (start 133.32 108.71) (end 131.48 110.55) (width 0.2) (layer "F.Cu") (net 18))
 (segment (start 131.48 110.55) (end 108.35 110.55) (width 0.2) (layer "F.Cu") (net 18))
 (segment (start 108.35 113.05) (end 109.627 113.05) (width 0.2) (layer "F.Cu") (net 17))
 (segment (start 109.627 113.05) (end 109.897 112.78) (width 0.2) (layer "F.Cu") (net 17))
 (segment (start 134.85 112.78) (end 135.86 113.79) (width 0.2) (layer "F.Cu") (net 17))
 (segment (start 109.897 112.78) (end 134.85 112.78) (width 0.2) (layer "F.Cu") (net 17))
 (segment (start 114.319 118.759) (end 118.07 122.51) (width 0.2) (layer "B.Cu") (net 13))
 (segment (start 117.84 111.547) (end 114.319 115.068) (width 0.2) (layer "B.Cu") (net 13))
 (segment (start 114.319 115.068) (end 114.319 118.759) (width 0.2) (layer "B.Cu") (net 13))
 (segment (start 117.84 106.64) (end 117.84 111.547) (width 0.2) (layer "B.Cu") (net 13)))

